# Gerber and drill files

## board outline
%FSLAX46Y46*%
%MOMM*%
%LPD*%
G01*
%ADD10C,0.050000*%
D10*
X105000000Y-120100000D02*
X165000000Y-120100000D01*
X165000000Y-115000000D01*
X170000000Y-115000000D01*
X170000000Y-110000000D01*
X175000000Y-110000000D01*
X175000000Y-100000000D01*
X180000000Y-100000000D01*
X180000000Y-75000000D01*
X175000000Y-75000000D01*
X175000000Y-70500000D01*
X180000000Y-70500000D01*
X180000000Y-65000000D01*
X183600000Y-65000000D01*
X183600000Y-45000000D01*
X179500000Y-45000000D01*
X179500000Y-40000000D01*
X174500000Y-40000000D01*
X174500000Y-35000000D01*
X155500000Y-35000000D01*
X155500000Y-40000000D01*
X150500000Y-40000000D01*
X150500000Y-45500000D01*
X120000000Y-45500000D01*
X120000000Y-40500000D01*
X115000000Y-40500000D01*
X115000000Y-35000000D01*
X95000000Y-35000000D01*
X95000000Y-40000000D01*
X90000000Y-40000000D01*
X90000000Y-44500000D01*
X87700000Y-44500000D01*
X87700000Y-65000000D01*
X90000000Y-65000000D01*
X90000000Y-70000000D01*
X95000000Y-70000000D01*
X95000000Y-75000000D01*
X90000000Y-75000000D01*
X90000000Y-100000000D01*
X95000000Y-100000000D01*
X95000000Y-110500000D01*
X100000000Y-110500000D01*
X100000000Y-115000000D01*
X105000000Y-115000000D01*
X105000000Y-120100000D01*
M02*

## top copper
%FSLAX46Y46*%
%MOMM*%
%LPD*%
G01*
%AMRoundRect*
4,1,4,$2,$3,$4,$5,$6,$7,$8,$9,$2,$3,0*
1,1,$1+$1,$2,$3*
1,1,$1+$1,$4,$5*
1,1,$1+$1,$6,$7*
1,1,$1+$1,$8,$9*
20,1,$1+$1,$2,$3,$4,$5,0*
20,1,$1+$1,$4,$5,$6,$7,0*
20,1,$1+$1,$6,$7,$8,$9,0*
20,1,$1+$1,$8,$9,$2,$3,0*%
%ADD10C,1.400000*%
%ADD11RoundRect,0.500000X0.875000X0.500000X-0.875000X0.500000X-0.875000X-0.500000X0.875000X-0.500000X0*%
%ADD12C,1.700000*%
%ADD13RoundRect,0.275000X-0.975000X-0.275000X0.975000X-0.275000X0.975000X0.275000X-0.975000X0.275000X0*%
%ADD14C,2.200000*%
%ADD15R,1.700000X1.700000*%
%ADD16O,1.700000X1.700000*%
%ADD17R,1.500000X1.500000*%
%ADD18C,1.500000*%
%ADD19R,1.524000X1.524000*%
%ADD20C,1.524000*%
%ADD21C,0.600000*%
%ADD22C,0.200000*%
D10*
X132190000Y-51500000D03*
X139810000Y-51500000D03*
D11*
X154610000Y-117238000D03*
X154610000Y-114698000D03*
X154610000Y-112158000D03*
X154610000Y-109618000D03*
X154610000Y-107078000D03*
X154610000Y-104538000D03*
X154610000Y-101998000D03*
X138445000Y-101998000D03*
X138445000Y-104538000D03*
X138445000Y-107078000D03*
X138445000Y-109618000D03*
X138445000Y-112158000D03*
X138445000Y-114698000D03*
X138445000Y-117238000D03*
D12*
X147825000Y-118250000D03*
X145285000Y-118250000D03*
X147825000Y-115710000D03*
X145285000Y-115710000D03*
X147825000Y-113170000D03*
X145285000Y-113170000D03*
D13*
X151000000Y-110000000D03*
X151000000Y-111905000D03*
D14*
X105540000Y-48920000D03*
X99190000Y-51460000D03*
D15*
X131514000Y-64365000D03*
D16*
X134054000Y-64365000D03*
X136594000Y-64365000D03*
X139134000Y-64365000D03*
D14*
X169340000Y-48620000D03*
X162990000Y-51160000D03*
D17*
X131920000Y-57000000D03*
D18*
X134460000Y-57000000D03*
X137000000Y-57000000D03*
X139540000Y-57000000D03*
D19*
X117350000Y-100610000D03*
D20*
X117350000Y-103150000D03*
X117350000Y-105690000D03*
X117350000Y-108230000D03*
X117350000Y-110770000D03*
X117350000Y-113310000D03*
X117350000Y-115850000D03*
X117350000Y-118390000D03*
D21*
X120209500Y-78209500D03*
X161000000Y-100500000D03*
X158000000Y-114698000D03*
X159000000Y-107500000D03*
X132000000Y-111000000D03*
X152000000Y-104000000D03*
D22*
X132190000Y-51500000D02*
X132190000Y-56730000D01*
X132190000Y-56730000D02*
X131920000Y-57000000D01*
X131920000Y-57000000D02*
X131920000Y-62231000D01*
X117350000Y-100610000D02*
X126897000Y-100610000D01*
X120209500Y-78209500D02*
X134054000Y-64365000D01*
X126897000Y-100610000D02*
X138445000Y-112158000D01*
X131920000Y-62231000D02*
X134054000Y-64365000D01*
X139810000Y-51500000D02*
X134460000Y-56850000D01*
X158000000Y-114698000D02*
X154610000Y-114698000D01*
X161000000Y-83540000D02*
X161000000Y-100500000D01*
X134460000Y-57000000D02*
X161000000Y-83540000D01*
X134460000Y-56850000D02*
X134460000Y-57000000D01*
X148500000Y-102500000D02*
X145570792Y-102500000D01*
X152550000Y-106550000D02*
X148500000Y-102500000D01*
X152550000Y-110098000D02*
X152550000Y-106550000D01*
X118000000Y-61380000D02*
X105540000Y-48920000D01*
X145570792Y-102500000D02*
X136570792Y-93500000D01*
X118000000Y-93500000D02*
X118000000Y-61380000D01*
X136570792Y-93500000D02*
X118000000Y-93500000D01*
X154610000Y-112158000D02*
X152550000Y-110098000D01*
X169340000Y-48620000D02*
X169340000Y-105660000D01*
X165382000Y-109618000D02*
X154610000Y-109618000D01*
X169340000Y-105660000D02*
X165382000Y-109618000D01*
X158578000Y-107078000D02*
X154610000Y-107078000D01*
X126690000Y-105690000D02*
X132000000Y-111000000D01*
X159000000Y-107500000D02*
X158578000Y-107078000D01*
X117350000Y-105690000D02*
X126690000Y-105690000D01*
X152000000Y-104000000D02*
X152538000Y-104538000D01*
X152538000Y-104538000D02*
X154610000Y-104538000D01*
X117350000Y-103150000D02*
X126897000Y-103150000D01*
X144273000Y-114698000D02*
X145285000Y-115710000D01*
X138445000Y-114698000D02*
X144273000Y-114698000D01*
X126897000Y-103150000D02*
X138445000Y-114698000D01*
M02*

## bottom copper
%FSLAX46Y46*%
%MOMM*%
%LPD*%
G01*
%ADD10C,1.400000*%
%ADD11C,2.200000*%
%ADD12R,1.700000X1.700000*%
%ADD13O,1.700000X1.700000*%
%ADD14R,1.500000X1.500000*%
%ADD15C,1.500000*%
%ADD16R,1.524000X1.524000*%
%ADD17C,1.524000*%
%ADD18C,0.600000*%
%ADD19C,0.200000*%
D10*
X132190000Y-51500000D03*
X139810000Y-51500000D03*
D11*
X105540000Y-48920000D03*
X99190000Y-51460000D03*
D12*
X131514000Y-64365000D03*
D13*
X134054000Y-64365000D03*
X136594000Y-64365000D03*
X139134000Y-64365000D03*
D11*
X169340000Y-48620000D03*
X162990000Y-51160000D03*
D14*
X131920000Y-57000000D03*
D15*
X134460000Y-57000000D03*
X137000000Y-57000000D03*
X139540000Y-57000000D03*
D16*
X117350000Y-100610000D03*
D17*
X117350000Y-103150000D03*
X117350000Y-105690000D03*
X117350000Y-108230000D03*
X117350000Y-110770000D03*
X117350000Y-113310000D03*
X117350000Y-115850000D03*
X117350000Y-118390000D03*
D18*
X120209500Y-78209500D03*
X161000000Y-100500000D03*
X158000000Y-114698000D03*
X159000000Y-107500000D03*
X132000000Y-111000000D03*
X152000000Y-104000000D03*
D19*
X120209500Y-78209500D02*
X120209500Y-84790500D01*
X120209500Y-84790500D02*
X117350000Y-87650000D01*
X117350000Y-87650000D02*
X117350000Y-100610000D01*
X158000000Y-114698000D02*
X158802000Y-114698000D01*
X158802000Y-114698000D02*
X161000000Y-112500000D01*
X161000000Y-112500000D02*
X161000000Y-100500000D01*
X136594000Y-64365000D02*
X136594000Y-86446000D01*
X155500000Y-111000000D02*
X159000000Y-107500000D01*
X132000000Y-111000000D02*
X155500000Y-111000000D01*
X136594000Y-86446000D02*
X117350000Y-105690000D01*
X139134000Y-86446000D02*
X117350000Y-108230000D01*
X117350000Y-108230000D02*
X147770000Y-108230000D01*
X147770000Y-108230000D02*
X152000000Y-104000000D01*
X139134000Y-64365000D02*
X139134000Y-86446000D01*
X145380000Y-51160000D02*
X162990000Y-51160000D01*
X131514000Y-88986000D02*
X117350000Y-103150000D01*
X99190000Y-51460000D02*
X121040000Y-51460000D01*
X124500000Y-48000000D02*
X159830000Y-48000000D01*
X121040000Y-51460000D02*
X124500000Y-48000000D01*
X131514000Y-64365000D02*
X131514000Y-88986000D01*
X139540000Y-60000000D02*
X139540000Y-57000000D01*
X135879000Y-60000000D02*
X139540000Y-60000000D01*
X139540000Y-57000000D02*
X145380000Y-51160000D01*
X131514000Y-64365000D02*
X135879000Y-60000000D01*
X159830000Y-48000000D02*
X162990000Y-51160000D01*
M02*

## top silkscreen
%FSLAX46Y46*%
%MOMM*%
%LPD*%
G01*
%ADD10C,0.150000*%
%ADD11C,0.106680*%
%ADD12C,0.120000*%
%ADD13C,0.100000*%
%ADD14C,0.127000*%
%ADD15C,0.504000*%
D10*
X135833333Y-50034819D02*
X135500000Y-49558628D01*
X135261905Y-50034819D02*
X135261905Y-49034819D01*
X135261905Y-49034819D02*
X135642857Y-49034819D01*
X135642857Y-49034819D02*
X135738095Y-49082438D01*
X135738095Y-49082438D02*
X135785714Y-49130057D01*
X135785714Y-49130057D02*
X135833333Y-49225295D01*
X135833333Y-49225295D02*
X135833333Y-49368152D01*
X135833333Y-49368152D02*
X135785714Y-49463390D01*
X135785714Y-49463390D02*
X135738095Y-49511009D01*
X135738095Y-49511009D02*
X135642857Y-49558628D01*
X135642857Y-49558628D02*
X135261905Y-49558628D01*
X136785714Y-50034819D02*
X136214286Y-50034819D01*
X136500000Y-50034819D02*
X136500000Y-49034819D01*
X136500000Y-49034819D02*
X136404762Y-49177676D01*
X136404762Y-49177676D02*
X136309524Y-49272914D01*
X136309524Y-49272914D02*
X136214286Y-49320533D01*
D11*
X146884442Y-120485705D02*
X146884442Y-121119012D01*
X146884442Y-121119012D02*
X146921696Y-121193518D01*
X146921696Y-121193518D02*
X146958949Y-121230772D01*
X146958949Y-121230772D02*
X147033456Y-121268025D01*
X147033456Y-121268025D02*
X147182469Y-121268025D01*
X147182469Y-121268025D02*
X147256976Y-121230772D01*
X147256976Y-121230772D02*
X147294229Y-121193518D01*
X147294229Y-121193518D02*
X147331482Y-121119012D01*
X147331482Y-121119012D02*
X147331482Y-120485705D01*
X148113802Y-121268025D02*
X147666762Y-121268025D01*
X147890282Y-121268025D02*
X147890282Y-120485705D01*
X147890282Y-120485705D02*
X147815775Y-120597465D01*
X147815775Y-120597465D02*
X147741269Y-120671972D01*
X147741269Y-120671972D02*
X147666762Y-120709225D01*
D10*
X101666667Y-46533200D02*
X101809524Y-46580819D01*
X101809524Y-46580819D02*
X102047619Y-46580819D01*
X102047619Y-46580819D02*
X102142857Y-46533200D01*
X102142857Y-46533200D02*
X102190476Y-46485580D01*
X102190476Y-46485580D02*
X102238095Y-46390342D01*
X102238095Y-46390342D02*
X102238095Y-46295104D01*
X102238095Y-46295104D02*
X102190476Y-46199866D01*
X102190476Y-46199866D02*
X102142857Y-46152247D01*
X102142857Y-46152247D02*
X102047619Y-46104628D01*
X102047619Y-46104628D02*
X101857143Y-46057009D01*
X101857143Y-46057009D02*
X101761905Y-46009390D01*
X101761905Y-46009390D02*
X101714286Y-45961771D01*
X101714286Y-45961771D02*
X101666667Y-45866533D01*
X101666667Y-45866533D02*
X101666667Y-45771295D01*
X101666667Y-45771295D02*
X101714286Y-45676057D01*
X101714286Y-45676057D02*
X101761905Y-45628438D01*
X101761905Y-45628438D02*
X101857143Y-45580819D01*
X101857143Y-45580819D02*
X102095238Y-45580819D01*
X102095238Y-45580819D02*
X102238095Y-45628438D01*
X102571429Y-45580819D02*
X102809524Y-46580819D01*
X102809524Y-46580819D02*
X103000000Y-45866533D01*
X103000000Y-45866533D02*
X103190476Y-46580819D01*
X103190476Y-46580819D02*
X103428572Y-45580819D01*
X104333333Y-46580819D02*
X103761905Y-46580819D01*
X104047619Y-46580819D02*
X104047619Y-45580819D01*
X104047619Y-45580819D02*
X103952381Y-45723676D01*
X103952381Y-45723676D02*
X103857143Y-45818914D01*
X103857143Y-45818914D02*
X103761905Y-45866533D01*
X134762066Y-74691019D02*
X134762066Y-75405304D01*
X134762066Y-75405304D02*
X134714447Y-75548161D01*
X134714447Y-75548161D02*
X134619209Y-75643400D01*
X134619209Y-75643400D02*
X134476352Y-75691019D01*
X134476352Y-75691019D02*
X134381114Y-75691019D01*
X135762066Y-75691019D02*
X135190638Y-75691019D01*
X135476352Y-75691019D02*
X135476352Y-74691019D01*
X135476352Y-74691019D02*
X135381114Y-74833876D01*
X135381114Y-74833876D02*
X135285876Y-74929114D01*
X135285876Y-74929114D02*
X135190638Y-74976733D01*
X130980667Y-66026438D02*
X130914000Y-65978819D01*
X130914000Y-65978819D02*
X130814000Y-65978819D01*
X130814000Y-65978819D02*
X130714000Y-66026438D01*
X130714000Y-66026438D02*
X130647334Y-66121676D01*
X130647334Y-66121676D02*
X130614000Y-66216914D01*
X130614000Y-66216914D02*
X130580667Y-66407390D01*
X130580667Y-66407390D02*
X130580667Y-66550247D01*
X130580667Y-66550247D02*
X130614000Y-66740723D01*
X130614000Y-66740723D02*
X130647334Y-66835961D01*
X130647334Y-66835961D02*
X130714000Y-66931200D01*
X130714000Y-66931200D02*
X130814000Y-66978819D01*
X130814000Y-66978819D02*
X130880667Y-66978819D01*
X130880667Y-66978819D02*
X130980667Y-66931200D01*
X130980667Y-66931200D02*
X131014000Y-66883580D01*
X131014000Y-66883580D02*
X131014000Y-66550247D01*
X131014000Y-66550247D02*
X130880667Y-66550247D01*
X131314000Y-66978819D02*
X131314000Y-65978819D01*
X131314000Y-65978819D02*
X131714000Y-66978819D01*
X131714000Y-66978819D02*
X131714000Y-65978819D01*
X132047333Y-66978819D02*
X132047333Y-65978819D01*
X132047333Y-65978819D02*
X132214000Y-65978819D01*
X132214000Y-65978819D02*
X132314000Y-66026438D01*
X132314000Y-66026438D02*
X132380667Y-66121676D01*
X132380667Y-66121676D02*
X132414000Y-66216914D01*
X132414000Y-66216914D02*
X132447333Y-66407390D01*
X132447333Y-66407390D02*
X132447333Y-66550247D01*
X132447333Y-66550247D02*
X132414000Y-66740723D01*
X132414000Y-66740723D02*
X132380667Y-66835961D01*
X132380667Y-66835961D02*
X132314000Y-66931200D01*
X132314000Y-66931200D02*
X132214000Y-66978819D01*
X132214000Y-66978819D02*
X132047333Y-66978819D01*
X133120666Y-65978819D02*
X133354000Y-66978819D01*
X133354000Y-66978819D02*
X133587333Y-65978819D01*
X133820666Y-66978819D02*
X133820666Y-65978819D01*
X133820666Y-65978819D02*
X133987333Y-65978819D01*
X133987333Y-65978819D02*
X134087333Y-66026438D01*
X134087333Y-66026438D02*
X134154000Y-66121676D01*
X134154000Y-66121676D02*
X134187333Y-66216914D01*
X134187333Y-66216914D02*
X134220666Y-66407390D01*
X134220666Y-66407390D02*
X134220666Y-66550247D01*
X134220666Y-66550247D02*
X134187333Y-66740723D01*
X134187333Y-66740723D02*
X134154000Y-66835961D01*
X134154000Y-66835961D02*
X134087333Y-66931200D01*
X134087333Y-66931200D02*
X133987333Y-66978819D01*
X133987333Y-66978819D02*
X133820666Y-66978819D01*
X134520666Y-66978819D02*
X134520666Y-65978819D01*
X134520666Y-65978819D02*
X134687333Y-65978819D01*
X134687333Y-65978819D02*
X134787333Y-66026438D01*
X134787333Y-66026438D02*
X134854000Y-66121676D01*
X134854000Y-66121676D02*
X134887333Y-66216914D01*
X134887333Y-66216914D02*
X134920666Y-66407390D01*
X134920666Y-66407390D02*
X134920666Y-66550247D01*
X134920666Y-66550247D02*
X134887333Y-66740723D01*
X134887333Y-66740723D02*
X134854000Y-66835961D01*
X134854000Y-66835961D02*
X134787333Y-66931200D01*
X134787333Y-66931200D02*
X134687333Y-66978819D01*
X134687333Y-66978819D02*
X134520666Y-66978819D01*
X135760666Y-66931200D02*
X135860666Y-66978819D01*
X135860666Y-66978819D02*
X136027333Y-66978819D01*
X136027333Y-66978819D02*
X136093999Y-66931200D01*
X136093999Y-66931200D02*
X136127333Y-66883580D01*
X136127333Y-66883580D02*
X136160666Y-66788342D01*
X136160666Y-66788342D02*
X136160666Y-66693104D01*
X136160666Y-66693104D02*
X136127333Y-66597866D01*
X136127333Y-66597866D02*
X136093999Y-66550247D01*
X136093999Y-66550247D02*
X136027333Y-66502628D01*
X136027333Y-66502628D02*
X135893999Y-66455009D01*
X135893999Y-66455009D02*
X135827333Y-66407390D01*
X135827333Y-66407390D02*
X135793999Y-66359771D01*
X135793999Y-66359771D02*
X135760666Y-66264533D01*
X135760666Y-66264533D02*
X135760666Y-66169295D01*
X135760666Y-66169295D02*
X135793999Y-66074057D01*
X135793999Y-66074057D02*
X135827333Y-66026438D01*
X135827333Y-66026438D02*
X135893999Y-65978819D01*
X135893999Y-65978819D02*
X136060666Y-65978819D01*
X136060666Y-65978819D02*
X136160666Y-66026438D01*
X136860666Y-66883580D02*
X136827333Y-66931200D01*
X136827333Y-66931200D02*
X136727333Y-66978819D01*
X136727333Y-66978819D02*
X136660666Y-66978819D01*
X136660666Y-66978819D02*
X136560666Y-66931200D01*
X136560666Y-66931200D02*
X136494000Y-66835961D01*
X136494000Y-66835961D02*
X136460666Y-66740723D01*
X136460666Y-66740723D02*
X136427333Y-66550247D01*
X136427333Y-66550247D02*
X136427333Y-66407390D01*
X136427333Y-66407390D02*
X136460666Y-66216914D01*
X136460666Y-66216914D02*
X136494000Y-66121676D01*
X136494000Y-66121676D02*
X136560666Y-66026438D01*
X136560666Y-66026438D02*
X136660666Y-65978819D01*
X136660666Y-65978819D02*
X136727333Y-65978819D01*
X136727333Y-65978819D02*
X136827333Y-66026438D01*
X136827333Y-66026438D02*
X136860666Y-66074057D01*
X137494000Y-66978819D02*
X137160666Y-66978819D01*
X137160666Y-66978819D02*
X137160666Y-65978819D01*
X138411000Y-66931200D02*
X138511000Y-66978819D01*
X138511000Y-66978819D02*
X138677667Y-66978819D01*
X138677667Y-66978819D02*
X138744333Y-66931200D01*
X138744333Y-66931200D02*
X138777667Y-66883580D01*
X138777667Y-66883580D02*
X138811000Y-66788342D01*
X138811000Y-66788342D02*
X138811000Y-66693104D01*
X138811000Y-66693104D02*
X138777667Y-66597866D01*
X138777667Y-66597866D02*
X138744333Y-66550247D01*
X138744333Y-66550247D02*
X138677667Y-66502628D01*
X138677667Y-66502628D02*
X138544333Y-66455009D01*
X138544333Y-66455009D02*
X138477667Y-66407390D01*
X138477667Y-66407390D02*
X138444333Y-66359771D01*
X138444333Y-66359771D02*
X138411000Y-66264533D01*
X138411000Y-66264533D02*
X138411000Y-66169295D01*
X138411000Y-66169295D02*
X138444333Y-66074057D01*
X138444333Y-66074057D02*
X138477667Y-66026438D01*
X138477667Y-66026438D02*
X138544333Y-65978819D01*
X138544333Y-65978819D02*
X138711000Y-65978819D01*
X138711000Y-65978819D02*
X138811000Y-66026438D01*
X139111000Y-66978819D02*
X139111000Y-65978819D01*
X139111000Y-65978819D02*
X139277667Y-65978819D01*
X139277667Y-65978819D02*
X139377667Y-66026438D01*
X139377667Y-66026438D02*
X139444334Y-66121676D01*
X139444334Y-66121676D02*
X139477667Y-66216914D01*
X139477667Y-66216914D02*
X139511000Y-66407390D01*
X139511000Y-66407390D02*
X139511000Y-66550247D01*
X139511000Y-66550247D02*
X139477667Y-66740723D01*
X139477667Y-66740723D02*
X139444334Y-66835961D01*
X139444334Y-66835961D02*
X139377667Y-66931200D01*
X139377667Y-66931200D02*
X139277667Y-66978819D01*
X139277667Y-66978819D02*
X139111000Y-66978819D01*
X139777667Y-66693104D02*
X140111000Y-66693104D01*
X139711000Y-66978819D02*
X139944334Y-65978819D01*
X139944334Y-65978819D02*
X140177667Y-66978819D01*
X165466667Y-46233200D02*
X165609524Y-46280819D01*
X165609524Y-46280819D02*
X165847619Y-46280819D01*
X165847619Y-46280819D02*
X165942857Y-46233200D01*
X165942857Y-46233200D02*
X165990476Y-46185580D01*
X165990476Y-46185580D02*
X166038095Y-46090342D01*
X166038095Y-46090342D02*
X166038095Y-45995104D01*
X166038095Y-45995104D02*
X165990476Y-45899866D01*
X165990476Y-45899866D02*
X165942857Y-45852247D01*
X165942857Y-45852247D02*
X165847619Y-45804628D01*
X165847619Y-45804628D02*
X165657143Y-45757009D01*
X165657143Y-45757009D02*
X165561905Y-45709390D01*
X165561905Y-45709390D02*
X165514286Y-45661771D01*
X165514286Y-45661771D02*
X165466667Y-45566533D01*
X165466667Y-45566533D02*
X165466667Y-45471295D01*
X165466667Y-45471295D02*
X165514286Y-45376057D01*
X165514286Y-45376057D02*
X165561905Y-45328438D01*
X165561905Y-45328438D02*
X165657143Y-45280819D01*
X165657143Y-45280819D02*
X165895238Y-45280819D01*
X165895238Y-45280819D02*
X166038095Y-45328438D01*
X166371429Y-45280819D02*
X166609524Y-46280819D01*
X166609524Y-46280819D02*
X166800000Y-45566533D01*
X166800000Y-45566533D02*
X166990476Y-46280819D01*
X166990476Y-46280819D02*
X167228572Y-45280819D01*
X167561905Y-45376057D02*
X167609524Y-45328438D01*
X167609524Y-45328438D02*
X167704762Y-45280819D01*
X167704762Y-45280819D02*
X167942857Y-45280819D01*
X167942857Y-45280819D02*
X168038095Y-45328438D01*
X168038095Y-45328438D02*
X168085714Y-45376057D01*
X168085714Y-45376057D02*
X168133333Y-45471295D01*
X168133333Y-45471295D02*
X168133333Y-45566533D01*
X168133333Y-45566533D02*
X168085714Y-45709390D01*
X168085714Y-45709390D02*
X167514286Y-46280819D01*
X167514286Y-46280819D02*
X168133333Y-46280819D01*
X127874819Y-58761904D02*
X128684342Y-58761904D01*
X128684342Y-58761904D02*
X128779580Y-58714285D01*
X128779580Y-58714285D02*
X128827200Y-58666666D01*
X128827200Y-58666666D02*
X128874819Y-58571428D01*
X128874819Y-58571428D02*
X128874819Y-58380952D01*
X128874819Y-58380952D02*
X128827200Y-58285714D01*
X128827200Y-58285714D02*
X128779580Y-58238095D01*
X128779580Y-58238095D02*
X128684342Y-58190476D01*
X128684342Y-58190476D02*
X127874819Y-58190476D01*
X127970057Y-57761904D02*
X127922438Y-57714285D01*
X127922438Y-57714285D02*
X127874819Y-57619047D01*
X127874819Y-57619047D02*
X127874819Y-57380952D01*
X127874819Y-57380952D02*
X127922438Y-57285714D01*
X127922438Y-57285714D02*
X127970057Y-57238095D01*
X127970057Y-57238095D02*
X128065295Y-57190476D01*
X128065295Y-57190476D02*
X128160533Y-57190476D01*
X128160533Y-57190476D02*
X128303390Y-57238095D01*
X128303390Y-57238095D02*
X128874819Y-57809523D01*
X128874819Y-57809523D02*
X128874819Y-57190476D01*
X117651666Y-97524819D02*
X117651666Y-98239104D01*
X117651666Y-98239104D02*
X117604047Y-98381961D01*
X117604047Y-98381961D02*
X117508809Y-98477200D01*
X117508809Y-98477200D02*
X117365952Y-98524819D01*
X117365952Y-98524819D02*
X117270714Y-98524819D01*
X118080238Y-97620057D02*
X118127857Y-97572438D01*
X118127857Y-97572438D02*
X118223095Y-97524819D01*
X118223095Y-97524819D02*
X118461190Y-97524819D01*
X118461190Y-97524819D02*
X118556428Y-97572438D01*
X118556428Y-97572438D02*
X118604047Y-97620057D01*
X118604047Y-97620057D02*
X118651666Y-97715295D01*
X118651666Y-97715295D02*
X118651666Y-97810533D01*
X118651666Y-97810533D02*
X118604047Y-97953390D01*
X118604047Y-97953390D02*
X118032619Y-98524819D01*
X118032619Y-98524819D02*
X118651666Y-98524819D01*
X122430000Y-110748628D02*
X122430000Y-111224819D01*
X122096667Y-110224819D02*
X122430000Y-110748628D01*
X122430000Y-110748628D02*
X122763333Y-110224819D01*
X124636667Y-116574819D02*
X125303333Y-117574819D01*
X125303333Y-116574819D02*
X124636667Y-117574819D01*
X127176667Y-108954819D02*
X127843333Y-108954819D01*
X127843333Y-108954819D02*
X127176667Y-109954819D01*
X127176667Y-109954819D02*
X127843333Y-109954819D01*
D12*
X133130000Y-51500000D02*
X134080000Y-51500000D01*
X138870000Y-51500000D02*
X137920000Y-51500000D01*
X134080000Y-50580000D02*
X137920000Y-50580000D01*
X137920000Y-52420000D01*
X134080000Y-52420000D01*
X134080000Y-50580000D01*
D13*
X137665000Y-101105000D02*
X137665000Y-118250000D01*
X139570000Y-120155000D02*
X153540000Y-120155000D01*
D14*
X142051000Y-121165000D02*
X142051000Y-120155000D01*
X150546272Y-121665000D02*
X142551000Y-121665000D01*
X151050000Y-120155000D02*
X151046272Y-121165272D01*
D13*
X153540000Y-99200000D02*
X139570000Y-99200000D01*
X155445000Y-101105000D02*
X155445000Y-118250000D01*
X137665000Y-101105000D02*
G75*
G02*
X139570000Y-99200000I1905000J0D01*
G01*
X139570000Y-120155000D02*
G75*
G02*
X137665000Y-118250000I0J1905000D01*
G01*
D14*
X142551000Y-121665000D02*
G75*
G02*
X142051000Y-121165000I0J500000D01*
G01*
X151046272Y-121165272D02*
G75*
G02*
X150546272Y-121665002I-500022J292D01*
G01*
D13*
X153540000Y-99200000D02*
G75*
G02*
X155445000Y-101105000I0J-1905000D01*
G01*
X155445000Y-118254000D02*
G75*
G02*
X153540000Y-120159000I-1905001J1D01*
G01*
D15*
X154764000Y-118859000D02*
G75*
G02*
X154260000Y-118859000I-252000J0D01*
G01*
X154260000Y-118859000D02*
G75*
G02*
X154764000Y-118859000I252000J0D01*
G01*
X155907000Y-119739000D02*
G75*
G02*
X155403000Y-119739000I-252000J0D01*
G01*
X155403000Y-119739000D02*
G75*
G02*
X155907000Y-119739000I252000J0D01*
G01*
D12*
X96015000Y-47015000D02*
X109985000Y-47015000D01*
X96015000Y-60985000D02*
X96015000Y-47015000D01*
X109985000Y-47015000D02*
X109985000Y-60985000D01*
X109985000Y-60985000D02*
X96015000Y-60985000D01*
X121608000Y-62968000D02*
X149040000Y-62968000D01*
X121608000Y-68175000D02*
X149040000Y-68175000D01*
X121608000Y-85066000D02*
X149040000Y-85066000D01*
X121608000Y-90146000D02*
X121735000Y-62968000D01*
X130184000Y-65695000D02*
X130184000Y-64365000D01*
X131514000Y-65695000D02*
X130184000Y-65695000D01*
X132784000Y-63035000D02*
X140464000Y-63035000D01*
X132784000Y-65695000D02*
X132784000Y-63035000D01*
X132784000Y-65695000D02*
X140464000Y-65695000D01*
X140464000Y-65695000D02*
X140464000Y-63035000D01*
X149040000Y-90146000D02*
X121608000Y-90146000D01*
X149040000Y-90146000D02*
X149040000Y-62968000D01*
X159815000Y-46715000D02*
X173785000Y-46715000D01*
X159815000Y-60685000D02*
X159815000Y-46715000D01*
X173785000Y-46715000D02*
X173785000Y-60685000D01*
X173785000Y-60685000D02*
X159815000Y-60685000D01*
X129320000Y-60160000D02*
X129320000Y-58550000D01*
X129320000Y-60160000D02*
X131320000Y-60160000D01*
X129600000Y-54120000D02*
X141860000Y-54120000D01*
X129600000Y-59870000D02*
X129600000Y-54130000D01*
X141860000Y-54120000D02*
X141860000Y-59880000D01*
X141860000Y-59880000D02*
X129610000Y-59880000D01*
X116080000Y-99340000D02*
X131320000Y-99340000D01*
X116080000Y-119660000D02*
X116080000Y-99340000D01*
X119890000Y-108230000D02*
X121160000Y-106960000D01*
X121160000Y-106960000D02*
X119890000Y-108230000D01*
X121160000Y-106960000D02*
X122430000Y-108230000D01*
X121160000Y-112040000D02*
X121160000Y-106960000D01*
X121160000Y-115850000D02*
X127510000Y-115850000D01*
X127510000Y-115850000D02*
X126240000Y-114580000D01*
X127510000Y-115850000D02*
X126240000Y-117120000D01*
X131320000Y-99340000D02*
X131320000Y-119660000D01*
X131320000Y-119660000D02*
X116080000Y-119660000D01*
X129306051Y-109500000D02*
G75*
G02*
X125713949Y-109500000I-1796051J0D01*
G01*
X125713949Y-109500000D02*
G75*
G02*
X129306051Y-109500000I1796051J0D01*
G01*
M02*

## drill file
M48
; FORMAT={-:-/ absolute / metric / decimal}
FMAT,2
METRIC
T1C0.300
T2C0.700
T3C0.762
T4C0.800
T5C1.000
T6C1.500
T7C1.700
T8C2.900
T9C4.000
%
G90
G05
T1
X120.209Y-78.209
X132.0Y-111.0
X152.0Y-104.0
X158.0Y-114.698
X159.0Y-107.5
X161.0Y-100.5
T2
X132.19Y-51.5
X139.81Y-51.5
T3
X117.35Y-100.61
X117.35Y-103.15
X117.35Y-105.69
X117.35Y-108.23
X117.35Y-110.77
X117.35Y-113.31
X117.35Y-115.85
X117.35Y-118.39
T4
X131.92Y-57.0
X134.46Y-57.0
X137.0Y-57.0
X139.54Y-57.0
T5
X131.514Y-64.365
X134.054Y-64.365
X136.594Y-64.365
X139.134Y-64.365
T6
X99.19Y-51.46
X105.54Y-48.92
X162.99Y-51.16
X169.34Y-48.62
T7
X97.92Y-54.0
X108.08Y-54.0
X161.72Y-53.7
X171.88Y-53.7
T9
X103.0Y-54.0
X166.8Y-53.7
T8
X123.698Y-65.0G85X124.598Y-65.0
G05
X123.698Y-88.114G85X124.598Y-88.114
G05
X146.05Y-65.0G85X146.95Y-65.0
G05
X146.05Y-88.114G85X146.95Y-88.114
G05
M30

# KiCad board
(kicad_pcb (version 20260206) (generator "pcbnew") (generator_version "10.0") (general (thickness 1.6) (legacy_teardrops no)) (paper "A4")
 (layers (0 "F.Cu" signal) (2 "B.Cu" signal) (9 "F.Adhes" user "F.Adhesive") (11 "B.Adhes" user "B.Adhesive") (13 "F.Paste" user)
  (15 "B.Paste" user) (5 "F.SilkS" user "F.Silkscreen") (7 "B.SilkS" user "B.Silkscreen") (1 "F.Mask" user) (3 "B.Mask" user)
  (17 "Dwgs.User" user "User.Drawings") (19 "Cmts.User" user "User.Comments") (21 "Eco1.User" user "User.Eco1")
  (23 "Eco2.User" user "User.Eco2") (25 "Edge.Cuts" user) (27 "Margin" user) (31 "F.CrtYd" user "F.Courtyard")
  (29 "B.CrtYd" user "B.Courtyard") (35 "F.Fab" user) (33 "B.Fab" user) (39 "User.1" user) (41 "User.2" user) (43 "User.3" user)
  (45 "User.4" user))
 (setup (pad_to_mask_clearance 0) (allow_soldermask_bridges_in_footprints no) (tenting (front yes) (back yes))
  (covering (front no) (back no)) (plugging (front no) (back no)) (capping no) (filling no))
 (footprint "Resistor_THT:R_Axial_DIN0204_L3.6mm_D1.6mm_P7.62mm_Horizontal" (layer "F.Cu") (at 132.19 51.5)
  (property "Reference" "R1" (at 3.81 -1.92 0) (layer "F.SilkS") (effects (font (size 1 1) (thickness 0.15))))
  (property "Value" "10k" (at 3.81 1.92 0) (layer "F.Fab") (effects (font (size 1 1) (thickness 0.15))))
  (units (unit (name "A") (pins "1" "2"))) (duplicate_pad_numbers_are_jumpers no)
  (fp_line (start 0.94 0) (end 1.89 0) (stroke (width 0.12) (type solid)) (layer "F.SilkS"))
  (fp_line (start 6.68 0) (end 5.73 0) (stroke (width 0.12) (type solid)) (layer "F.SilkS"))
  (fp_rect (start 1.89 -0.92) (end 5.73 0.92) (stroke (width 0.12) (type solid)) (fill no) (layer "F.SilkS"))
  (pad "1" thru_hole circle (at 0 0) (size 1.4 1.4) (drill 0.7) (layers "*.Cu" "*.Mask") (remove_unused_layers no) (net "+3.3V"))
  (pad "2" thru_hole circle (at 7.62 0) (size 1.4 1.4) (drill 0.7) (layers "*.Cu" "*.Mask") (remove_unused_layers no) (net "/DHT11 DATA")))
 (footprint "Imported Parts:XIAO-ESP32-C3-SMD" (layer "F.Cu") (at 155.445 99.118 180)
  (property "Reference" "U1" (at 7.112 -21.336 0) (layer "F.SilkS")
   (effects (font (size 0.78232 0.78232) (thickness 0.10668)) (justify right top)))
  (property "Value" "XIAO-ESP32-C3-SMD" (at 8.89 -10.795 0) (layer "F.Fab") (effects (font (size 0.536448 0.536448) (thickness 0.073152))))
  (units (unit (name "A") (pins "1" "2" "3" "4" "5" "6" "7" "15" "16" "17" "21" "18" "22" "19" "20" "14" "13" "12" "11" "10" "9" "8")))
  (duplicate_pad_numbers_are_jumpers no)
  (fp_line (start 17.78 -1.987) (end 17.78 -19.132) (stroke (width 0.1) (type solid)) (layer "F.SilkS"))
  (fp_line (start 15.875 -21.037) (end 1.905 -21.037) (stroke (width 0.1) (type solid)) (layer "F.SilkS"))
  (fp_line (start 13.394 -22.047) (end 13.394 -21.037) (stroke (width 0.127) (type solid)) (layer "F.SilkS"))
  (fp_line (start 4.898728 -22.547) (end 12.894 -22.547) (stroke (width 0.127) (type solid)) (layer "F.SilkS"))
  (fp_line (start 4.395 -21.037) (end 4.398728 -22.047272) (stroke (width 0.127) (type solid)) (layer "F.SilkS"))
  (fp_line (start 1.905 -0.082) (end 15.875 -0.082) (stroke (width 0.1) (type solid)) (layer "F.SilkS"))
  (fp_line (start 0 -1.987) (end 0 -19.132) (stroke (width 0.1) (type solid)) (layer "F.SilkS"))
  (fp_arc (start 17.78 -1.987) (mid 17.222038 -0.639962) (end 15.875 -0.082) (stroke (width 0.1) (type solid)) (layer "F.SilkS"))
  (fp_arc (start 15.875 -21.037) (mid 17.222038 -20.479038) (end 17.78 -19.132) (stroke (width 0.1) (type solid)) (layer "F.SilkS"))
  (fp_arc (start 12.894 -22.547) (mid 13.247553 -22.400553) (end 13.394 -22.047) (stroke (width 0.127) (type default)) (layer "F.SilkS"))
  (fp_arc (start 4.398728 -22.047272) (mid 4.545272 -22.40064) (end 4.898728 -22.547) (stroke (width 0.127) (type default))
   (layer "F.SilkS"))
  (fp_arc (start 1.905 -0.082) (mid 0.557962 -0.639962) (end 0 -1.987) (stroke (width 0.1) (type solid)) (layer "F.SilkS"))
  (fp_arc (start 0 -19.136) (mid 0.557962 -20.483038) (end 1.905 -21.041) (stroke (width 0.1) (type solid)) (layer "F.SilkS"))
  (fp_circle (center 0.933 -19.741) (end 0.933 -19.995) (stroke (width 0.5) (type solid)) (fill yes) (layer "F.SilkS"))
  (fp_circle (center -0.21 -20.621) (end -0.21 -20.875) (stroke (width 0.5) (type solid)) (fill yes) (layer "F.SilkS"))
  (pad "1" smd roundrect (at 0.835 -18.12 180) (size 2.75 2) (layers "F.Cu" "F.Mask" "F.Paste") (roundrect_rratio 0.25)
   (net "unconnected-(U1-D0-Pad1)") (solder_mask_margin 0.0508) (thermal_bridge_angle 45))
  (pad "2" smd roundrect (at 0.835 -15.58 180) (size 2.75 2) (layers "F.Cu" "F.Mask" "F.Paste") (roundrect_rratio 0.25) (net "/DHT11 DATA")
   (solder_mask_margin 0.0508) (thermal_bridge_angle 45))
  (pad "3" smd roundrect (at 0.835 -13.04 180) (size 2.75 2) (layers "F.Cu" "F.Mask" "F.Paste") (roundrect_rratio 0.25) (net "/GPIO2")
   (solder_mask_margin 0.0508) (thermal_bridge_angle 45))
  (pad "4" smd roundrect (at 0.835 -10.5 180) (size 2.75 2) (layers "F.Cu" "F.Mask" "F.Paste") (roundrect_rratio 0.25) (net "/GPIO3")
   (solder_mask_margin 0.0508) (thermal_bridge_angle 45))
  (pad "5" smd roundrect (at 0.835 -7.96 180) (size 2.75 2) (layers "F.Cu" "F.Mask" "F.Paste") (roundrect_rratio 0.25) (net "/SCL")
   (solder_mask_margin 0.0508) (thermal_bridge_angle 45))
  (pad "6" smd roundrect (at 0.835 -5.42 180) (size 2.75 2) (layers "F.Cu" "F.Mask" "F.Paste") (roundrect_rratio 0.25) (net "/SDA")
   (solder_mask_margin 0.0508) (thermal_bridge_angle 45))
  (pad "7" smd roundrect (at 0.835 -2.88 180) (size 2.75 2) (layers "F.Cu" "F.Mask" "F.Paste") (roundrect_rratio 0.25)
   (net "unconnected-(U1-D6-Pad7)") (solder_mask_margin 0.0508) (thermal_bridge_angle 45))
  (pad "8" smd roundrect (at 17 -2.88 180) (size 2.75 2) (layers "F.Cu" "F.Mask" "F.Paste") (roundrect_rratio 0.25)
   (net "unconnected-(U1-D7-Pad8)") (solder_mask_margin 0.0508) (thermal_bridge_angle 45))
  (pad "9" smd roundrect (at 17 -5.42 180) (size 2.75 2) (layers "F.Cu" "F.Mask" "F.Paste") (roundrect_rratio 0.25)
   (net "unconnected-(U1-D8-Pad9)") (solder_mask_margin 0.0508) (thermal_bridge_angle 45))
  (pad "10" smd roundrect (at 17 -7.96 180) (size 2.75 2) (layers "F.Cu" "F.Mask" "F.Paste") (roundrect_rratio 0.25)
   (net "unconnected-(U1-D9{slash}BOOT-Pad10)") (solder_mask_margin 0.0508) (thermal_bridge_angle 45))
  (pad "11" smd roundrect (at 17 -10.5 180) (size 2.75 2) (layers "F.Cu" "F.Mask" "F.Paste") (roundrect_rratio 0.25)
   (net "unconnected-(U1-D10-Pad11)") (solder_mask_margin 0.0508) (thermal_bridge_angle 45))
  (pad "12" smd roundrect (at 17 -13.04 180) (size 2.75 2) (layers "F.Cu" "F.Mask" "F.Paste") (roundrect_rratio 0.25) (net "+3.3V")
   (solder_mask_margin 0.0508) (thermal_bridge_angle 45))
  (pad "13" smd roundrect (at 17 -15.58 180) (size 2.75 2) (layers "F.Cu" "F.Mask" "F.Paste") (roundrect_rratio 0.25) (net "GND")
   (solder_mask_margin 0.0508) (thermal_bridge_angle 45))
  (pad "14" smd roundrect (at 17 -18.12 180) (size 2.75 2) (layers "F.Cu" "F.Mask" "F.Paste") (roundrect_rratio 0.25) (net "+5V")
   (solder_mask_margin 0.0508) (thermal_bridge_angle 45))
  (pad "15" smd circle (at 7.62 -19.132 180) (size 1.7 1.7) (layers "F.Cu" "F.Mask" "F.Paste") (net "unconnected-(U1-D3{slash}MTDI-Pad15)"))
  (pad "16" smd circle (at 10.16 -19.132 180) (size 1.7 1.7) (layers "F.Cu" "F.Mask" "F.Paste") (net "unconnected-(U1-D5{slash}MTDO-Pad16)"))
  (pad "17" smd circle (at 7.62 -16.592 180) (size 1.7 1.7) (layers "F.Cu" "F.Mask" "F.Paste") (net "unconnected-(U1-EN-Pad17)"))
  (pad "18" smd circle (at 10.16 -16.592 180) (size 1.7 1.7) (layers "F.Cu" "F.Mask" "F.Paste") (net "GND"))
  (pad "19" smd circle (at 7.62 -14.052 180) (size 1.7 1.7) (layers "F.Cu" "F.Mask" "F.Paste") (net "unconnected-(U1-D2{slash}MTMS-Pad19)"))
  (pad "20" smd circle (at 10.16 -14.052 180) (size 1.7 1.7) (layers "F.Cu" "F.Mask" "F.Paste") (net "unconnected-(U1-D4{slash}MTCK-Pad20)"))
  (pad "21" smd roundrect (at 4.445 -10.882) (size 2.5 1.1) (layers "F.Cu" "F.Mask" "F.Paste") (roundrect_rratio 0.25)
   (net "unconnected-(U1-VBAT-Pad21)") (thermal_bridge_angle 45))
  (pad "22" smd roundrect (at 4.445 -12.787) (size 2.5 1.1) (layers "F.Cu" "F.Mask" "F.Paste") (roundrect_rratio 0.25)
   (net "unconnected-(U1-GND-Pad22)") (thermal_bridge_angle 45)))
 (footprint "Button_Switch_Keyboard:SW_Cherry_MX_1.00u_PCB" (layer "F.Cu") (at 105.54 48.92)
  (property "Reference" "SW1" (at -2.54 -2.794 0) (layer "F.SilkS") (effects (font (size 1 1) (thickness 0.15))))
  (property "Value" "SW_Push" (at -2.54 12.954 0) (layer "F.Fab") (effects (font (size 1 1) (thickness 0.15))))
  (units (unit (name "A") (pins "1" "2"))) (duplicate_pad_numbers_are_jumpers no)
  (fp_line (start -9.525 -1.905) (end 4.445 -1.905) (stroke (width 0.12) (type solid)) (layer "F.SilkS"))
  (fp_line (start -9.525 12.065) (end -9.525 -1.905) (stroke (width 0.12) (type solid)) (layer "F.SilkS"))
  (fp_line (start 4.445 -1.905) (end 4.445 12.065) (stroke (width 0.12) (type solid)) (layer "F.SilkS"))
  (fp_line (start 4.445 12.065) (end -9.525 12.065) (stroke (width 0.12) (type solid)) (layer "F.SilkS"))
  (pad "" np_thru_hole circle (at -7.62 5.08) (size 1.7 1.7) (drill 1.7) (layers "*.Cu" "*.Mask"))
  (pad "" np_thru_hole circle (at -2.54 5.08) (size 4 4) (drill 4) (layers "*.Cu" "*.Mask"))
  (pad "" np_thru_hole circle (at 2.54 5.08) (size 1.7 1.7) (drill 1.7) (layers "*.Cu" "*.Mask"))
  (pad "1" thru_hole circle (at 0 0) (size 2.2 2.2) (drill 1.5) (layers "*.Cu" "*.Mask") (remove_unused_layers no) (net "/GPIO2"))
  (pad "2" thru_hole circle (at -6.35 2.54) (size 2.2 2.2) (drill 1.5) (layers "*.Cu" "*.Mask") (remove_unused_layers no) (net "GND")))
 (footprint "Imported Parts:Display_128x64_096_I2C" (layer "F.Cu") (at 135.324 64.365)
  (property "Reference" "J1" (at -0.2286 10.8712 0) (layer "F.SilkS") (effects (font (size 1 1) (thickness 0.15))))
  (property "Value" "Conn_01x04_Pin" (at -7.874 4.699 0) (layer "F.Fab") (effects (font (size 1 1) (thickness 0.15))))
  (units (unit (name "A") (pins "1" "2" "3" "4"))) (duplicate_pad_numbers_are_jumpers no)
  (fp_line (start -13.716 -1.397) (end 13.716 -1.397) (stroke (width 0.12) (type solid)) (layer "F.SilkS"))
  (fp_line (start -13.716 3.81) (end 13.716 3.81) (stroke (width 0.12) (type solid)) (layer "F.SilkS"))
  (fp_line (start -13.716 20.701) (end 13.716 20.701) (stroke (width 0.12) (type solid)) (layer "F.SilkS"))
  (fp_line (start -13.716 25.781) (end -13.589 -1.397) (stroke (width 0.12) (type solid)) (layer "F.SilkS"))
  (fp_line (start -5.14 1.33) (end -5.14 0) (stroke (width 0.12) (type solid)) (layer "F.SilkS"))
  (fp_line (start -3.81 1.33) (end -5.14 1.33) (stroke (width 0.12) (type solid)) (layer "F.SilkS"))
  (fp_line (start -2.54 -1.33) (end 5.14 -1.33) (stroke (width 0.12) (type solid)) (layer "F.SilkS"))
  (fp_line (start -2.54 1.33) (end -2.54 -1.33) (stroke (width 0.12) (type solid)) (layer "F.SilkS"))
  (fp_line (start -2.54 1.33) (end 5.14 1.33) (stroke (width 0.12) (type solid)) (layer "F.SilkS"))
  (fp_line (start 5.14 1.33) (end 5.14 -1.33) (stroke (width 0.12) (type solid)) (layer "F.SilkS"))
  (fp_line (start 13.716 25.781) (end -13.716 25.781) (stroke (width 0.12) (type solid)) (layer "F.SilkS"))
  (fp_line (start 13.716 25.781) (end 13.716 -1.397) (stroke (width 0.12) (type solid)) (layer "F.SilkS"))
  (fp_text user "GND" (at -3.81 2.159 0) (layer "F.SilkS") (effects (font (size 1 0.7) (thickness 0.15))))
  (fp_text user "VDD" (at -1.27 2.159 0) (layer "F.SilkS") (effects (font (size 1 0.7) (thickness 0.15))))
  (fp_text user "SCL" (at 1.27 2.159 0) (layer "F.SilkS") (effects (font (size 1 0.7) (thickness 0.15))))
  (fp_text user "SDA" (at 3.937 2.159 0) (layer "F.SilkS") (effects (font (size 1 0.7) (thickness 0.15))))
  (pad "" np_thru_hole oval (at -11.176 0.635) (size 3.8 2.9) (drill oval 3.8 2.9) (layers "*.Cu" "*.Mask"))
  (pad "" np_thru_hole oval (at -11.176 23.749) (size 3.8 2.9) (drill oval 3.8 2.9) (layers "*.Cu" "*.Mask"))
  (pad "" np_thru_hole oval (at 11.176 0.635) (size 3.8 2.9) (drill oval 3.8 2.9) (layers "*.Cu" "*.Mask"))
  (pad "" np_thru_hole oval (at 11.176 23.749) (size 3.8 2.9) (drill oval 3.8 2.9) (layers "*.Cu" "*.Mask"))
  (pad "1" thru_hole rect (at -3.81 0 90) (size 1.7 1.7) (drill 1) (layers "*.Cu" "*.Mask") (remove_unused_layers no) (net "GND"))
  (pad "2" thru_hole oval (at -1.27 0 90) (size 1.7 1.7) (drill 1) (layers "*.Cu" "*.Mask") (remove_unused_layers no) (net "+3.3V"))
  (pad "3" thru_hole oval (at 1.27 0 90) (size 1.7 1.7) (drill 1) (layers "*.Cu" "*.Mask") (remove_unused_layers no) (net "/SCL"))
  (pad "4" thru_hole oval (at 3.81 0 90) (size 1.7 1.7) (drill 1) (layers "*.Cu" "*.Mask") (remove_unused_layers no) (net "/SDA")))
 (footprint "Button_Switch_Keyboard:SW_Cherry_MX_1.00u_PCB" (layer "F.Cu") (at 169.34 48.62)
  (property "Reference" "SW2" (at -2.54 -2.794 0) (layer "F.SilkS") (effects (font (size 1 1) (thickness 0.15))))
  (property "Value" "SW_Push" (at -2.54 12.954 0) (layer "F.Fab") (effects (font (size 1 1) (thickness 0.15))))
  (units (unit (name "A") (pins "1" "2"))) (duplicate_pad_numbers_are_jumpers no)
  (fp_line (start -9.525 -1.905) (end 4.445 -1.905) (stroke (width 0.12) (type solid)) (layer "F.SilkS"))
  (fp_line (start -9.525 12.065) (end -9.525 -1.905) (stroke (width 0.12) (type solid)) (layer "F.SilkS"))
  (fp_line (start 4.445 -1.905) (end 4.445 12.065) (stroke (width 0.12) (type solid)) (layer "F.SilkS"))
  (fp_line (start 4.445 12.065) (end -9.525 12.065) (stroke (width 0.12) (type solid)) (layer "F.SilkS"))
  (pad "" np_thru_hole circle (at -7.62 5.08) (size 1.7 1.7) (drill 1.7) (layers "*.Cu" "*.Mask"))
  (pad "" np_thru_hole circle (at -2.54 5.08) (size 4 4) (drill 4) (layers "*.Cu" "*.Mask"))
  (pad "" np_thru_hole circle (at 2.54 5.08) (size 1.7 1.7) (drill 1.7) (layers "*.Cu" "*.Mask"))
  (pad "1" thru_hole circle (at 0 0) (size 2.2 2.2) (drill 1.5) (layers "*.Cu" "*.Mask") (remove_unused_layers no) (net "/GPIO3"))
  (pad "2" thru_hole circle (at -6.35 2.54) (size 2.2 2.2) (drill 1.5) (layers "*.Cu" "*.Mask") (remove_unused_layers no) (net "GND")))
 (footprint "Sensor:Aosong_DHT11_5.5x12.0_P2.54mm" (layer "F.Cu") (at 131.92 57 90)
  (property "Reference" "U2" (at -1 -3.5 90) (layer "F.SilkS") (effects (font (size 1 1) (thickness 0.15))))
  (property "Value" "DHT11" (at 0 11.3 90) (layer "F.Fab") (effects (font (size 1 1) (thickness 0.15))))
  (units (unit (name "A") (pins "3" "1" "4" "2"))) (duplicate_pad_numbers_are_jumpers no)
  (fp_line (start -3.16 -2.6) (end -1.55 -2.6) (stroke (width 0.12) (type solid)) (layer "F.SilkS"))
  (fp_line (start -3.16 -2.6) (end -3.16 -0.6) (stroke (width 0.12) (type solid)) (layer "F.SilkS"))
  (fp_line (start 2.88 -2.32) (end 2.88 9.94) (stroke (width 0.12) (type solid)) (layer "F.SilkS"))
  (fp_line (start -2.87 -2.32) (end 2.87 -2.32) (stroke (width 0.12) (type solid)) (layer "F.SilkS"))
  (fp_line (start 2.88 9.94) (end -2.88 9.94) (stroke (width 0.12) (type solid)) (layer "F.SilkS"))
  (fp_line (start -2.88 9.94) (end -2.88 -2.31) (stroke (width 0.12) (type solid)) (layer "F.SilkS"))
  (pad "1" thru_hole rect (at 0 0 90) (size 1.5 1.5) (drill 0.8) (layers "*.Cu" "*.Mask") (remove_unused_layers no) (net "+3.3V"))
  (pad "2" thru_hole circle (at 0 2.54 90) (size 1.5 1.5) (drill 0.8) (layers "*.Cu" "*.Mask") (remove_unused_layers no) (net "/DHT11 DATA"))
  (pad "3" thru_hole circle (at 0 5.08 90) (size 1.5 1.5) (drill 0.8) (layers "*.Cu" "*.Mask") (remove_unused_layers no)
   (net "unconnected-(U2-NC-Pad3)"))
  (pad "4" thru_hole circle (at 0 7.62 90) (size 1.5 1.5) (drill 0.8) (layers "*.Cu" "*.Mask") (remove_unused_layers no) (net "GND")))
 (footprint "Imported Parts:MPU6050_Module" (layer "F.Cu") (at 117.35 100.61)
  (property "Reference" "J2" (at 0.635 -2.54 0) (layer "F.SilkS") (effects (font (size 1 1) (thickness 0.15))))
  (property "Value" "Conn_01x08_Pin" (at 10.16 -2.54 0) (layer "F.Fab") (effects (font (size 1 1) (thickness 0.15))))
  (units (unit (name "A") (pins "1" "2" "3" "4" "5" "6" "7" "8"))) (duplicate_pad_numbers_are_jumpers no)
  (fp_line (start -1.27 -1.27) (end 13.97 -1.27) (stroke (width 0.12) (type solid)) (layer "F.SilkS"))
  (fp_line (start -1.27 19.05) (end -1.27 -1.27) (stroke (width 0.12) (type solid)) (layer "F.SilkS"))
  (fp_line (start 2.54 7.62) (end 3.81 6.35) (stroke (width 0.12) (type solid)) (layer "F.SilkS"))
  (fp_line (start 3.81 6.35) (end 2.54 7.62) (stroke (width 0.12) (type solid)) (layer "F.SilkS"))
  (fp_line (start 3.81 6.35) (end 5.08 7.62) (stroke (width 0.12) (type solid)) (layer "F.SilkS"))
  (fp_line (start 3.81 11.43) (end 3.81 6.35) (stroke (width 0.12) (type solid)) (layer "F.SilkS"))
  (fp_line (start 3.81 15.24) (end 10.16 15.24) (stroke (width 0.12) (type solid)) (layer "F.SilkS"))
  (fp_line (start 10.16 15.24) (end 8.89 13.97) (stroke (width 0.12) (type solid)) (layer "F.SilkS"))
  (fp_line (start 10.16 15.24) (end 8.89 16.51) (stroke (width 0.12) (type solid)) (layer "F.SilkS"))
  (fp_line (start 13.97 -1.27) (end 13.97 19.05) (stroke (width 0.12) (type solid)) (layer "F.SilkS"))
  (fp_line (start 13.97 19.05) (end -1.27 19.05) (stroke (width 0.12) (type solid)) (layer "F.SilkS"))
  (fp_circle (center 10.16 8.89) (end 8.89 7.62) (stroke (width 0.12) (type solid)) (fill no) (layer "F.SilkS"))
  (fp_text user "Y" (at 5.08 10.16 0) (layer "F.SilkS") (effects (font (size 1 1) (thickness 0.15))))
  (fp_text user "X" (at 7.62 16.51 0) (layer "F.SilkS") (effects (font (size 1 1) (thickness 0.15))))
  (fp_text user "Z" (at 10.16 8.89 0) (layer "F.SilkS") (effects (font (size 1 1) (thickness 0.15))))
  (pad "1" thru_hole rect (at 0 0) (size 1.524 1.524) (drill 0.762) (layers "*.Cu" "*.Mask") (remove_unused_layers no) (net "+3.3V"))
  (pad "2" thru_hole circle (at 0 2.54) (size 1.524 1.524) (drill 0.762) (layers "*.Cu" "*.Mask") (remove_unused_layers no) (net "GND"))
  (pad "3" thru_hole circle (at 0 5.08) (size 1.524 1.524) (drill 0.762) (layers "*.Cu" "*.Mask") (remove_unused_layers no) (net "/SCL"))
  (pad "4" thru_hole circle (at 0 7.62) (size 1.524 1.524) (drill 0.762) (layers "*.Cu" "*.Mask") (remove_unused_layers no) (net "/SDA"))
  (pad "5" thru_hole circle (at 0 10.16) (size 1.524 1.524) (drill 0.762) (layers "*.Cu" "*.Mask") (remove_unused_layers no)
   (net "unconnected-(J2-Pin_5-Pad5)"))
  (pad "6" thru_hole circle (at 0 12.7) (size 1.524 1.524) (drill 0.762) (layers "*.Cu" "*.Mask") (remove_unused_layers no)
   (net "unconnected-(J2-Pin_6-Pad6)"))
  (pad "7" thru_hole circle (at 0 15.24) (size 1.524 1.524) (drill 0.762) (layers "*.Cu" "*.Mask") (remove_unused_layers no)
   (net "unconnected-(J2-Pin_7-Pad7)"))
  (pad "8" thru_hole circle (at 0 17.78) (size 1.524 1.524) (drill 0.762) (layers "*.Cu" "*.Mask") (remove_unused_layers no)
   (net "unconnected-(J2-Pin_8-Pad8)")))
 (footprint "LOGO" (layer "B.Cu") (at 146.41959 88.78751 180)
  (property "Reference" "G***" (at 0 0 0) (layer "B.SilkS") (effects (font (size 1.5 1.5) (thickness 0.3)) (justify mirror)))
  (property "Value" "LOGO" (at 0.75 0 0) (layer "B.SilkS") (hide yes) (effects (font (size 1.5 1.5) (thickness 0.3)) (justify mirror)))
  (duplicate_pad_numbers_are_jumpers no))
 (gr_poly
  (pts (xy 105 120.1) (xy 165 120.1) (xy 165 115) (xy 170 115) (xy 170 110) (xy 175 110) (xy 175 100) (xy 180 100) (xy 180 75) (xy 175 75)
   (xy 175 70.5) (xy 180 70.5) (xy 180 65) (xy 183.6 65) (xy 183.6 45) (xy 179.5 45) (xy 179.5 40) (xy 174.5 40) (xy 174.5 35) (xy 155.5 35)
   (xy 155.5 40) (xy 150.5 40) (xy 150.5 45.5) (xy 120 45.5) (xy 120 40.5) (xy 115 40.5) (xy 115 35) (xy 95 35) (xy 95 40) (xy 90 40)
   (xy 90 44.5) (xy 87.7 44.5) (xy 87.7 65) (xy 90 65) (xy 90 70) (xy 95 70) (xy 95 75) (xy 90 75) (xy 90 100) (xy 95 100) (xy 95 110.5)
   (xy 100 110.5) (xy 100 115) (xy 105 115))
  (stroke (width 0.05) (type solid)) (fill no) (layer "Edge.Cuts"))
 (segment (start 132.19 51.5) (end 132.19 56.73) (width 0.2) (layer "F.Cu") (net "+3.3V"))
 (segment (start 132.19 56.73) (end 131.92 57) (width 0.2) (layer "F.Cu") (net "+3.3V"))
 (segment (start 131.92 57) (end 131.92 62.231) (width 0.2) (layer "F.Cu") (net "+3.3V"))
 (segment (start 117.35 100.61) (end 126.897 100.61) (width 0.2) (layer "F.Cu") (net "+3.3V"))
 (segment (start 120.2095 78.2095) (end 134.054 64.365) (width 0.2) (layer "F.Cu") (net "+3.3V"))
 (segment (start 126.897 100.61) (end 138.445 112.158) (width 0.2) (layer "F.Cu") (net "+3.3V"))
 (segment (start 131.92 62.231) (end 134.054 64.365) (width 0.2) (layer "F.Cu") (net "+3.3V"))
 (via (at 120.2095 78.2095) (size 0.6) (drill 0.3) (layers "F.Cu" "B.Cu") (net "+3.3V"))
 (segment (start 120.2095 78.2095) (end 120.2095 84.7905) (width 0.2) (layer "B.Cu") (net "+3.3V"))
 (segment (start 120.2095 84.7905) (end 117.35 87.65) (width 0.2) (layer "B.Cu") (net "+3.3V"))
 (segment (start 117.35 87.65) (end 117.35 100.61) (width 0.2) (layer "B.Cu") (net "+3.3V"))
 (segment (start 139.81 51.5) (end 134.46 56.85) (width 0.2) (layer "F.Cu") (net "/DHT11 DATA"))
 (segment (start 158 114.698) (end 154.61 114.698) (width 0.2) (layer "F.Cu") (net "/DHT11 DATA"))
 (segment (start 161 83.54) (end 161 100.5) (width 0.2) (layer "F.Cu") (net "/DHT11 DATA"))
 (segment (start 134.46 57) (end 161 83.54) (width 0.2) (layer "F.Cu") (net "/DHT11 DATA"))
 (segment (start 134.46 56.85) (end 134.46 57) (width 0.2) (layer "F.Cu") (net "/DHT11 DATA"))
 (via (at 161 100.5) (size 0.6) (drill 0.3) (layers "F.Cu" "B.Cu") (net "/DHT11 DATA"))
 (via (at 158 114.698) (size 0.6) (drill 0.3) (layers "F.Cu" "B.Cu") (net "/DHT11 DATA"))
 (segment (start 158 114.698) (end 158.802 114.698) (width 0.2) (layer "B.Cu") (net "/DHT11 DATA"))
 (segment (start 158.802 114.698) (end 161 112.5) (width 0.2) (layer "B.Cu") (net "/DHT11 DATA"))
 (segment (start 161 112.5) (end 161 100.5) (width 0.2) (layer "B.Cu") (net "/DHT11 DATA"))
 (segment (start 148.5 102.5) (end 145.570792 102.5) (width 0.2) (layer "F.Cu") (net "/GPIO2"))
 (segment (start 152.55 106.55) (end 148.5 102.5) (width 0.2) (layer "F.Cu") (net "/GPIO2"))
 (segment (start 152.55 110.098) (end 152.55 106.55) (width 0.2) (layer "F.Cu") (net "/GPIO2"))
 (segment (start 118 61.38) (end 105.54 48.92) (width 0.2) (layer "F.Cu") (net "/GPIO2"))
 (segment (start 145.570792 102.5) (end 136.570792 93.5) (width 0.2) (layer "F.Cu") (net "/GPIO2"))
 (segment (start 118 93.5) (end 118 61.38) (width 0.2) (layer "F.Cu") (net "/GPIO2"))
 (segment (start 136.570792 93.5) (end 118 93.5) (width 0.2) (layer "F.Cu") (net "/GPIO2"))
 (segment (start 154.61 112.158) (end 152.55 110.098) (width 0.2) (layer "F.Cu") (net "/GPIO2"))
 (segment (start 169.34 48.62) (end 169.34 105.66) (width 0.2) (layer "F.Cu") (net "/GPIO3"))
 (segment (start 165.382 109.618) (end 154.61 109.618) (width 0.2) (layer "F.Cu") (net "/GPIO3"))
 (segment (start 169.34 105.66) (end 165.382 109.618) (width 0.2) (layer "F.Cu") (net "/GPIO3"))
 (segment (start 158.578 107.078) (end 154.61 107.078) (width 0.2) (layer "F.Cu") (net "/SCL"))
 (segment (start 126.69 105.69) (end 132 111) (width 0.2) (layer "F.Cu") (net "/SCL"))
 (segment (start 159 107.5) (end 158.578 107.078) (width 0.2) (layer "F.Cu") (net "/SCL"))
 (segment (start 117.35 105.69) (end 126.69 105.69) (width 0.2) (layer "F.Cu") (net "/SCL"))
 (via (at 159 107.5) (size 0.6) (drill 0.3) (layers "F.Cu" "B.Cu") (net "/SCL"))
 (via (at 132 111) (size 0.6) (drill 0.3) (layers "F.Cu" "B.Cu") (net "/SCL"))
 (segment (start 136.594 64.365) (end 136.594 86.446) (width 0.2) (layer "B.Cu") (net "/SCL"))
 (segment (start 155.5 111) (end 159 107.5) (width 0.2) (layer "B.Cu") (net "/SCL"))
 (segment (start 132 111) (end 155.5 111) (width 0.2) (layer "B.Cu") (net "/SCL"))
 (segment (start 136.594 86.446) (end 117.35 105.69) (width 0.2) (layer "B.Cu") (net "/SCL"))
 (segment (start 152 104) (end 152.538 104.538) (width 0.2) (layer "F.Cu") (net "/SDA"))
 (segment (start 152.538 104.538) (end 154.61 104.538) (width 0.2) (layer "F.Cu") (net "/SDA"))
 (via (at 152 104) (size 0.6) (drill 0.3) (layers "F.Cu" "B.Cu") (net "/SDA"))
 (segment (start 139.134 86.446) (end 117.35 108.23) (width 0.2) (layer "B.Cu") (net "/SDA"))
 (segment (start 117.35 108.23) (end 147.77 108.23) (width 0.2) (layer "B.Cu") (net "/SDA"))
 (segment (start 147.77 108.23) (end 152 104) (width 0.2) (layer "B.Cu") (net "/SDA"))
 (segment (start 139.134 64.365) (end 139.134 86.446) (width 0.2) (layer "B.Cu") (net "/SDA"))
 (segment (start 117.35 103.15) (end 126.897 103.15) (width 0.2) (layer "F.Cu") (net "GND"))
 (segment (start 144.273 114.698) (end 145.285 115.71) (width 0.2) (layer "F.Cu") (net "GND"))
 (segment (start 138.445 114.698) (end 144.273 114.698) (width 0.2) (layer "F.Cu") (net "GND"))
 (segment (start 126.897 103.15) (end 138.445 114.698) (width 0.2) (layer "F.Cu") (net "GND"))
 (segment (start 145.38 51.16) (end 162.99 51.16) (width 0.2) (layer "B.Cu") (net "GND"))
 (segment (start 131.514 88.986) (end 117.35 103.15) (width 0.2) (layer "B.Cu") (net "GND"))
 (segment (start 99.19 51.46) (end 121.04 51.46) (width 0.2) (layer "B.Cu") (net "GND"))
 (segment (start 124.5 48) (end 159.83 48) (width 0.2) (layer "B.Cu") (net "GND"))
 (segment (start 121.04 51.46) (end 124.5 48) (width 0.2) (layer "B.Cu") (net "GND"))
 (segment (start 131.514 64.365) (end 131.514 88.986) (width 0.2) (layer "B.Cu") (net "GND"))
 (segment (start 139.54 60) (end 139.54 57) (width 0.2) (layer "B.Cu") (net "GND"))
 (segment (start 135.879 60) (end 139.54 60) (width 0.2) (layer "B.Cu") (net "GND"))
 (segment (start 139.54 57) (end 145.38 51.16) (width 0.2) (layer "B.Cu") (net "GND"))
 (segment (start 131.514 64.365) (end 135.879 60) (width 0.2) (layer "B.Cu") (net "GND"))
 (segment (start 159.83 48) (end 162.99 51.16) (width 0.2) (layer "B.Cu") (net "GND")))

